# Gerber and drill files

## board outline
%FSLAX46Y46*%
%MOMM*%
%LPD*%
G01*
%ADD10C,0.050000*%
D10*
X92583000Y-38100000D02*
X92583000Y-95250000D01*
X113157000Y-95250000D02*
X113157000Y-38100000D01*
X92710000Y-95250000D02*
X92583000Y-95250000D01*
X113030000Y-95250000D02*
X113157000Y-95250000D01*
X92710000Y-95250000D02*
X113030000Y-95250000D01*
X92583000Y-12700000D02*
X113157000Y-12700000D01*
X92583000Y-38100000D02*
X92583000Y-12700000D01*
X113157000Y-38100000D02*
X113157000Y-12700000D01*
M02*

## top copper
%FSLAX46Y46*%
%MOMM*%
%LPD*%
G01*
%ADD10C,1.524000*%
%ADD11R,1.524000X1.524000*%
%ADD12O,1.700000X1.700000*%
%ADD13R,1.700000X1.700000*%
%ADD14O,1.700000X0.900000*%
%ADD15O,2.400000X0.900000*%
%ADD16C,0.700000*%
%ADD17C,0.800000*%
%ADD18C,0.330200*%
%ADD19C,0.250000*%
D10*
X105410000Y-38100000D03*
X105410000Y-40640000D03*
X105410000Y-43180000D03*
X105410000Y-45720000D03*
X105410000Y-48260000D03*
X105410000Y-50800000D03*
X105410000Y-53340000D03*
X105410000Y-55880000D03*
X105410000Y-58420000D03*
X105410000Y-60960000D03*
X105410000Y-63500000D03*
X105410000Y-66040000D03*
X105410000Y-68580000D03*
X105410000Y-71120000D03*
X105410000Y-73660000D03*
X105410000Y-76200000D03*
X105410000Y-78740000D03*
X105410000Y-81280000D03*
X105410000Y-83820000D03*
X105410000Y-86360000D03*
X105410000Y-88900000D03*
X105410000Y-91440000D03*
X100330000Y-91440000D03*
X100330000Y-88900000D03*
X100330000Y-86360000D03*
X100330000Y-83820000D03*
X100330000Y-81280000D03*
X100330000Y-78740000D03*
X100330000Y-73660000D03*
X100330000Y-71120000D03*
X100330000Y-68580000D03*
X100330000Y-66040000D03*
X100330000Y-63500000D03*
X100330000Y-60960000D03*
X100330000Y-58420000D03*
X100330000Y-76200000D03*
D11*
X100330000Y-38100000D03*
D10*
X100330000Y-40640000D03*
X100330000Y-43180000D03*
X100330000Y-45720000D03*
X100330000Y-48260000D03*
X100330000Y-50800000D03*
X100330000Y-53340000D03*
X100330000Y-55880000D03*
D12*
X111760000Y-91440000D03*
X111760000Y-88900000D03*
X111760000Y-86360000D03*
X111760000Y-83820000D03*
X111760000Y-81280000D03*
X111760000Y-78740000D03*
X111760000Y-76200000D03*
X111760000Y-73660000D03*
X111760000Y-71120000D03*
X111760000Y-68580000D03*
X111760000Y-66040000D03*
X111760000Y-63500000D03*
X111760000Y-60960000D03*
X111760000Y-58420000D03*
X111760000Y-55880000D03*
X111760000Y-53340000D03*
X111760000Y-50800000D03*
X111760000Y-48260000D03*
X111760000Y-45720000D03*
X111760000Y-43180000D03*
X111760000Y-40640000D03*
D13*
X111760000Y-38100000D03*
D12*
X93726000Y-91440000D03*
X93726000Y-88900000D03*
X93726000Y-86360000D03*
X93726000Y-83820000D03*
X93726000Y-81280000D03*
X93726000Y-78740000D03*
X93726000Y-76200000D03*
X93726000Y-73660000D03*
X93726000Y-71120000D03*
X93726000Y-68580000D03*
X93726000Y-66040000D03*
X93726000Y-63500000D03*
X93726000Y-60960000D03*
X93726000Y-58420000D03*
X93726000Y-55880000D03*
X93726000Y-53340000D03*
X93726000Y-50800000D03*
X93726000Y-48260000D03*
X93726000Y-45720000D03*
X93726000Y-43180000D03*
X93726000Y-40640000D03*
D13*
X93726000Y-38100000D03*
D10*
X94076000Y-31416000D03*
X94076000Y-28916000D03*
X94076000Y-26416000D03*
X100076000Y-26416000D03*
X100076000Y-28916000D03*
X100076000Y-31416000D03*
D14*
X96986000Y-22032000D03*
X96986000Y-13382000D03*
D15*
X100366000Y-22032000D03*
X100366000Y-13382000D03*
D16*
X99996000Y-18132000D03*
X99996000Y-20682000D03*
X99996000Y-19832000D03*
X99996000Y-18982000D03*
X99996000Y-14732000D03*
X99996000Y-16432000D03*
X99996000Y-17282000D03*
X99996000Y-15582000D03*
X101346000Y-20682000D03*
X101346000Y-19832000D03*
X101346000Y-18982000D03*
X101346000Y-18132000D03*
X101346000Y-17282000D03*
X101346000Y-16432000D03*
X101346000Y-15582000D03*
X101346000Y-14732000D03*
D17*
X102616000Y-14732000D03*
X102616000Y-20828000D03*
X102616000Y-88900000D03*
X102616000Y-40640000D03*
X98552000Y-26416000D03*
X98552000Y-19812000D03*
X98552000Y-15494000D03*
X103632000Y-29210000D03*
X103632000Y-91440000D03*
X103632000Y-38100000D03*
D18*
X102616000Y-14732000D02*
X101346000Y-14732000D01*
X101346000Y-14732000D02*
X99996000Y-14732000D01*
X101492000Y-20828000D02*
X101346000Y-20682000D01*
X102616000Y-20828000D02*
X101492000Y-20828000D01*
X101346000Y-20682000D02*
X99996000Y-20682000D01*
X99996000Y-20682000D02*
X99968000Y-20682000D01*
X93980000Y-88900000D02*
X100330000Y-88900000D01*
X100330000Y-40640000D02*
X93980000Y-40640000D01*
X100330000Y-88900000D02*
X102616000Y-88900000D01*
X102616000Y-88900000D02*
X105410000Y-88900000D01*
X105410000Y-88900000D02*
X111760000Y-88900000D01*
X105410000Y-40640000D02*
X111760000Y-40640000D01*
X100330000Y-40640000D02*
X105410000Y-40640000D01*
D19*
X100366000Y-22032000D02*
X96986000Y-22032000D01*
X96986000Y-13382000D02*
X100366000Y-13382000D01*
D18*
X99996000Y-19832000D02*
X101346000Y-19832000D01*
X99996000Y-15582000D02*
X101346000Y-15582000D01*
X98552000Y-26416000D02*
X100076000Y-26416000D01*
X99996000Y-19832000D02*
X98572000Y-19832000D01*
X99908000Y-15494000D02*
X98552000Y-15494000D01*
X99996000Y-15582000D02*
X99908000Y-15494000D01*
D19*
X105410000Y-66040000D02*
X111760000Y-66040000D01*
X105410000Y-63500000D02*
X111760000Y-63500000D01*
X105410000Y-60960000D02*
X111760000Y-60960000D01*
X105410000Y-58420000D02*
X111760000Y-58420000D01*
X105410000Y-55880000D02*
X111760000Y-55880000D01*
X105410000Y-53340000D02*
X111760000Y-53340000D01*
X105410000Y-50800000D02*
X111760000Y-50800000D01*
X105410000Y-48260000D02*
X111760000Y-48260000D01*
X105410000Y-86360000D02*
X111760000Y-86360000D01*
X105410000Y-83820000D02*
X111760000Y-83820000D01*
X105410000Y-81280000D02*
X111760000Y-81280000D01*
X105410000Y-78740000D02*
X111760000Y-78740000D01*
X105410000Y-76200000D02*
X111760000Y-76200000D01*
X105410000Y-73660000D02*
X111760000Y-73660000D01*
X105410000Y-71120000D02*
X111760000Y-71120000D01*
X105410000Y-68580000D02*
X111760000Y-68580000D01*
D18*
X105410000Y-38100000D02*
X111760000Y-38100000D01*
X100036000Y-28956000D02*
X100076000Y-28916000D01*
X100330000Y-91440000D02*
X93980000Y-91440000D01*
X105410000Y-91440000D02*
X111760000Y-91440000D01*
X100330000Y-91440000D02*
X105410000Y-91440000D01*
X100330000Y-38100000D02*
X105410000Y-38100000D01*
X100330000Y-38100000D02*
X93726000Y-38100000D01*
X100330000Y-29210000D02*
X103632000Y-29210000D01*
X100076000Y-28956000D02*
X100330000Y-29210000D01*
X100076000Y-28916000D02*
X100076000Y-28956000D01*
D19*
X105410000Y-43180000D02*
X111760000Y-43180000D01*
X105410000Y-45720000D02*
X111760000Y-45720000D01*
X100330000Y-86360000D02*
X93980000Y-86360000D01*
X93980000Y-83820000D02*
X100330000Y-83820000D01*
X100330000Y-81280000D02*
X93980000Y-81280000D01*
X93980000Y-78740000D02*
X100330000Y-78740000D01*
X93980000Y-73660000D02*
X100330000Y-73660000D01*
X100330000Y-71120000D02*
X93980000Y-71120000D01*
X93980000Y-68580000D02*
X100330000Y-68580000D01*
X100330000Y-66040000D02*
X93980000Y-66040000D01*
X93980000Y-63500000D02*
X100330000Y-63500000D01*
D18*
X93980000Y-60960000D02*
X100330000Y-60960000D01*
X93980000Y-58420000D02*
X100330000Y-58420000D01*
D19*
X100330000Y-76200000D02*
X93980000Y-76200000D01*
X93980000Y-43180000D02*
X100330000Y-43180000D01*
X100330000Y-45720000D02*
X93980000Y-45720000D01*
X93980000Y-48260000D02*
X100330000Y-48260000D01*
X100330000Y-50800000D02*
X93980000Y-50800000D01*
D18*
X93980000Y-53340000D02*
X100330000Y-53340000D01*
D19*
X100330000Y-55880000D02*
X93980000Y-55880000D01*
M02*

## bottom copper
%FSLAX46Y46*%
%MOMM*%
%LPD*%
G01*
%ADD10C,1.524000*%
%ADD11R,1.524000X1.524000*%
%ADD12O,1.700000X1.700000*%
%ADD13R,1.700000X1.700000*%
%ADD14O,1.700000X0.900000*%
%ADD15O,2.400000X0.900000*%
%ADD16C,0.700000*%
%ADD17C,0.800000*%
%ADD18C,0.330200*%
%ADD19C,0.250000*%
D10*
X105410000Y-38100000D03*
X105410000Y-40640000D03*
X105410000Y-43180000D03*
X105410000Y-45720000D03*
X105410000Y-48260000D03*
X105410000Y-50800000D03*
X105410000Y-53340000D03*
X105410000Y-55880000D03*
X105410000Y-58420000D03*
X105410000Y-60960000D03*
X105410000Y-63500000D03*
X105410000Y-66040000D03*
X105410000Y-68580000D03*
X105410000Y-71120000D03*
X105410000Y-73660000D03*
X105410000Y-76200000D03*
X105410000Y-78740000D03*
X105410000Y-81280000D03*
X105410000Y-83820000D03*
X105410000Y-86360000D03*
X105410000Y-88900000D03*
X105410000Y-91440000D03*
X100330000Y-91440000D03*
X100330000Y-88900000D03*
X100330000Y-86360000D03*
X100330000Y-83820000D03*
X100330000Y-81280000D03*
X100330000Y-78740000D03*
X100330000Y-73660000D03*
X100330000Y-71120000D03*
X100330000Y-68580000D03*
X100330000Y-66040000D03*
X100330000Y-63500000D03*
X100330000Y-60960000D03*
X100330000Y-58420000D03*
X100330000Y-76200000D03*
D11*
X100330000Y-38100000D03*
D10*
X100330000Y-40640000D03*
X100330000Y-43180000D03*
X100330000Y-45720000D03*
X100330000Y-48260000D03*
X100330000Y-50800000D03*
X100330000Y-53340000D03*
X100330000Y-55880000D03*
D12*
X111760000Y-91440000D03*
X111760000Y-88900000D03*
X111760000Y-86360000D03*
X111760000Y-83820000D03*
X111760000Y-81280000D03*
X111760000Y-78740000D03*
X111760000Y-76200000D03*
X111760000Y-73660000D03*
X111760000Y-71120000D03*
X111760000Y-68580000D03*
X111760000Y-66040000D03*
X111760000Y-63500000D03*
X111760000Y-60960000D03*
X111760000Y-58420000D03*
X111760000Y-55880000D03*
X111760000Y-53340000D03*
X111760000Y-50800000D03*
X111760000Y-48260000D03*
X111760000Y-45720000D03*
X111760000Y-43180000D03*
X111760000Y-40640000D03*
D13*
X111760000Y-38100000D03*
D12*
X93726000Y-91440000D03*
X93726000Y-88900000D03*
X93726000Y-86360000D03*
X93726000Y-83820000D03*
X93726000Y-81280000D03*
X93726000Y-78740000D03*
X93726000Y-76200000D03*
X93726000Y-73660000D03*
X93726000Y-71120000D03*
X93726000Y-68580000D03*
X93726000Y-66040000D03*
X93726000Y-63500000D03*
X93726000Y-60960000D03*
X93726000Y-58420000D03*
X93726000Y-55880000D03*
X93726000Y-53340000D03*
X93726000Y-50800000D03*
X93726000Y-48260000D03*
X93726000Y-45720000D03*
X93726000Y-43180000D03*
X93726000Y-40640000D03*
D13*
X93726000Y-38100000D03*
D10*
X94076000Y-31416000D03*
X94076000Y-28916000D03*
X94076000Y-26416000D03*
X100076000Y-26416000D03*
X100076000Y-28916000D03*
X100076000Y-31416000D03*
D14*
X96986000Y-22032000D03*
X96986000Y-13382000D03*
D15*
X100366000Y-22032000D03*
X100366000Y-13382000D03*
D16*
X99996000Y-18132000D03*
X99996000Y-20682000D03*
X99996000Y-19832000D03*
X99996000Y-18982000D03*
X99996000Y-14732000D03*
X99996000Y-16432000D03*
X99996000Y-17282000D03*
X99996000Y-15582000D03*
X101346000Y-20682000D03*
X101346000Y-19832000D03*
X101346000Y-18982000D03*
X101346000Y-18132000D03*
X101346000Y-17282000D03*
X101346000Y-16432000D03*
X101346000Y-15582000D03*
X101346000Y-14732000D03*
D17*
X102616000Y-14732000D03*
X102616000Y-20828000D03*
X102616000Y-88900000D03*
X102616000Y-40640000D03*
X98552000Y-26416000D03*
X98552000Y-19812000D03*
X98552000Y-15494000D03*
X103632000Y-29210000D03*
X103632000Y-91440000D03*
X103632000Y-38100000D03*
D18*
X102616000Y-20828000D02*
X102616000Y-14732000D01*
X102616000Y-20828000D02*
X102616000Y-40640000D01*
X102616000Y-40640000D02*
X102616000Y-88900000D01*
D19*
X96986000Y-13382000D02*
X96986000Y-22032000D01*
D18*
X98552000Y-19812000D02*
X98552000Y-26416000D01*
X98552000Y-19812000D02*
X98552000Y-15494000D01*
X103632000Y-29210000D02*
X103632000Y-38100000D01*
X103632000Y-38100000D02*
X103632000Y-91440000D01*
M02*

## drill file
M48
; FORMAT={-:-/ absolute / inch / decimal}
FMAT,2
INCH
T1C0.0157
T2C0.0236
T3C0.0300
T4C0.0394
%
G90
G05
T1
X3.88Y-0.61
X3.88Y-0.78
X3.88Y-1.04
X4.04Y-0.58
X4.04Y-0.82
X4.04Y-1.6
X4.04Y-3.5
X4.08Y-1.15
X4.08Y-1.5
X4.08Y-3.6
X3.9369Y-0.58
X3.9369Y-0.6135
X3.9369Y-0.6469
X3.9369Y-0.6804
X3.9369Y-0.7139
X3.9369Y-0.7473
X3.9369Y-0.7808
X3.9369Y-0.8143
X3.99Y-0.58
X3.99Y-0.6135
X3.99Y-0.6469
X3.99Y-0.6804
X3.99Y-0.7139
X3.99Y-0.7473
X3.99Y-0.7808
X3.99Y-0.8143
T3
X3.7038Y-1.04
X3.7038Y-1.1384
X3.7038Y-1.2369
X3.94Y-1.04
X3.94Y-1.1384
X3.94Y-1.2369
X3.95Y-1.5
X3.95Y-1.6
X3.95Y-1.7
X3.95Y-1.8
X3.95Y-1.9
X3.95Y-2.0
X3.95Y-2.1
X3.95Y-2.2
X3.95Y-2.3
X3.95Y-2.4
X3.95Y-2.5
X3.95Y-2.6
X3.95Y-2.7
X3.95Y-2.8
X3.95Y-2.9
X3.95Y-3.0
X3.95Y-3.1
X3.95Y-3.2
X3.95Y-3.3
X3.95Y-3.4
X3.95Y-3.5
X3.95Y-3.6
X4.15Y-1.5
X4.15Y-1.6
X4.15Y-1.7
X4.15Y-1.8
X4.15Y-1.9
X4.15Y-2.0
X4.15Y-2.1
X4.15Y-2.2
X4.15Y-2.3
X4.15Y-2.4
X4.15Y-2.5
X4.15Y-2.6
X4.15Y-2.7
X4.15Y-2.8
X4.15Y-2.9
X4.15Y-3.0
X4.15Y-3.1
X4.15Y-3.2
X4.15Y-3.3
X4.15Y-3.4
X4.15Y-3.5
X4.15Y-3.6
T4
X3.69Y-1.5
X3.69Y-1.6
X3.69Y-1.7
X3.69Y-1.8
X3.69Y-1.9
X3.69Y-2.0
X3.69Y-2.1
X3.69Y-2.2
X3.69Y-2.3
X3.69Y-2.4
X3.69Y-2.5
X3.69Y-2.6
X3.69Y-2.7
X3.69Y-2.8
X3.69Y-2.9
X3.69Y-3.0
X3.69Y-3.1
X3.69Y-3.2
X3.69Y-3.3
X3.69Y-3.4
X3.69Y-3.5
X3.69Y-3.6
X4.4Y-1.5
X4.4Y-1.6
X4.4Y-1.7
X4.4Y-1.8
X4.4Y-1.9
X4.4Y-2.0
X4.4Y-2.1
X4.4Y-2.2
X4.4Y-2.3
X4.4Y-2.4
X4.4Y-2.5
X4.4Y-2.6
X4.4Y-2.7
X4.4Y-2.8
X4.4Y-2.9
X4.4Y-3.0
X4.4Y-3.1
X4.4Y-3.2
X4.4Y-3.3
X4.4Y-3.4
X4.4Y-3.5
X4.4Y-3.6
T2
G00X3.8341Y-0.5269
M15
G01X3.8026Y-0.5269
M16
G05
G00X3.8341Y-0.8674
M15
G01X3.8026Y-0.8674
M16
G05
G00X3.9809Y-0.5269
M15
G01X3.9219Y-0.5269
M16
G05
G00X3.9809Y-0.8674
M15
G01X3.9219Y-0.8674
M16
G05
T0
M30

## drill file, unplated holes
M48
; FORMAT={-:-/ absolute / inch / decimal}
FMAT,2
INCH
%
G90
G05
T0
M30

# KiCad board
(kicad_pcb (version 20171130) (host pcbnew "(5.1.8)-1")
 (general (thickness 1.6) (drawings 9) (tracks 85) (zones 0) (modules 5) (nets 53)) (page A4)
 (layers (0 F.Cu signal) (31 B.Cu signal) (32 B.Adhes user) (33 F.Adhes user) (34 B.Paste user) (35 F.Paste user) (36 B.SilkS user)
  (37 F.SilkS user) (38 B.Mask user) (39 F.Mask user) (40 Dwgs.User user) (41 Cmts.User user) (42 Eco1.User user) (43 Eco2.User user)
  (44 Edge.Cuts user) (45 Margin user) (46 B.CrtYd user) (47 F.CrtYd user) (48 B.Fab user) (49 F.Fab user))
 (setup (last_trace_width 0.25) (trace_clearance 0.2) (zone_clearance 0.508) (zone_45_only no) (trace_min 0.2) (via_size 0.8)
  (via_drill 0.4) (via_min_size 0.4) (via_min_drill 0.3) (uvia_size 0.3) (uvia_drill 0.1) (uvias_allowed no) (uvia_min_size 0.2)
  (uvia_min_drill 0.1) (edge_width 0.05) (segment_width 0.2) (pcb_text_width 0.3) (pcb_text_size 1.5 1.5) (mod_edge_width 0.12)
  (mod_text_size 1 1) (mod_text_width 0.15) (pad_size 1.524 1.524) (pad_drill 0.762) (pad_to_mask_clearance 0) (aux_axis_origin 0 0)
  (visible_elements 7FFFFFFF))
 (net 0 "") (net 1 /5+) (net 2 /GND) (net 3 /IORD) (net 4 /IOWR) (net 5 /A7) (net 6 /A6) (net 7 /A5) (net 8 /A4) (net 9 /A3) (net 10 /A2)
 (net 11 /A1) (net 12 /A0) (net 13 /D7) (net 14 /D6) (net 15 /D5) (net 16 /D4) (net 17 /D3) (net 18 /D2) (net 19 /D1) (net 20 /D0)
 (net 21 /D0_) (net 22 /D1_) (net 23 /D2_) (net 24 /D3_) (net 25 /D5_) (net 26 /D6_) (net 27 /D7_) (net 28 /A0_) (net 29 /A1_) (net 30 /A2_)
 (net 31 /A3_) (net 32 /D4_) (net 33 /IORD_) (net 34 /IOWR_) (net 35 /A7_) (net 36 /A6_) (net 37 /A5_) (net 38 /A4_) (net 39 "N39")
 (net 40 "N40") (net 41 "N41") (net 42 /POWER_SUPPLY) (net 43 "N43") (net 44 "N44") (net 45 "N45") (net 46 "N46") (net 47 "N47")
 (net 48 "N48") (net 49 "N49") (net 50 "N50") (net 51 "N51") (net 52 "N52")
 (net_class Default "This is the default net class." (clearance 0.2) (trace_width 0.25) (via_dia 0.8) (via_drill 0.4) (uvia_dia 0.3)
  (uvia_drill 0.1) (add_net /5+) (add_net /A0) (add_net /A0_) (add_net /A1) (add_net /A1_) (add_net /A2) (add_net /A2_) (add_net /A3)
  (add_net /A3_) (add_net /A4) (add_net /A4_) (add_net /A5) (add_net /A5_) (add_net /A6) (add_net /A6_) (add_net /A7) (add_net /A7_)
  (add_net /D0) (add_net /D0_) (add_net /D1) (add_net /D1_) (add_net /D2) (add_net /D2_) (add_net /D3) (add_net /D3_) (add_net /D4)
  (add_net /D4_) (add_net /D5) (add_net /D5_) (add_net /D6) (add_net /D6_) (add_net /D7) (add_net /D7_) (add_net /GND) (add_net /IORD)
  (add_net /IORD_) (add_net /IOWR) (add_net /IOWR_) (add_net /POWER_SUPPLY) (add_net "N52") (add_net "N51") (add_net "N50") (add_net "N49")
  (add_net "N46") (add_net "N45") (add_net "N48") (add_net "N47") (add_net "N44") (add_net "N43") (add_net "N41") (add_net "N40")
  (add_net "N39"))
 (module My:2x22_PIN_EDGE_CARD (layer F.Cu) (at 100.33 38.1)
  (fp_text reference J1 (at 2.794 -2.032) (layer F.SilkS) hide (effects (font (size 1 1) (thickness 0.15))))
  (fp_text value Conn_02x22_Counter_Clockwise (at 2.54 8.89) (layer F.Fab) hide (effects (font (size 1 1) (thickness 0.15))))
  (pad 44 thru_hole circle (at 5.08 0) (size 1.524 1.524) (drill 0.762) (layers *.Cu *.Mask) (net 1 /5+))
  (pad 43 thru_hole circle (at 5.08 2.54) (size 1.524 1.524) (drill 0.762) (layers *.Cu *.Mask) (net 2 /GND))
  (pad 42 thru_hole circle (at 5.08 5.08) (size 1.524 1.524) (drill 0.762) (layers *.Cu *.Mask) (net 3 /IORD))
  (pad 41 thru_hole circle (at 5.08 7.62) (size 1.524 1.524) (drill 0.762) (layers *.Cu *.Mask) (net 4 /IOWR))
  (pad 40 thru_hole circle (at 5.08 10.16) (size 1.524 1.524) (drill 0.762) (layers *.Cu *.Mask) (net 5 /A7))
  (pad 39 thru_hole circle (at 5.08 12.7) (size 1.524 1.524) (drill 0.762) (layers *.Cu *.Mask) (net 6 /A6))
  (pad 38 thru_hole circle (at 5.08 15.24) (size 1.524 1.524) (drill 0.762) (layers *.Cu *.Mask) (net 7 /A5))
  (pad 37 thru_hole circle (at 5.08 17.78) (size 1.524 1.524) (drill 0.762) (layers *.Cu *.Mask) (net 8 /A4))
  (pad 36 thru_hole circle (at 5.08 20.32) (size 1.524 1.524) (drill 0.762) (layers *.Cu *.Mask) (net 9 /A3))
  (pad 35 thru_hole circle (at 5.08 22.86) (size 1.524 1.524) (drill 0.762) (layers *.Cu *.Mask) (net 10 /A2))
  (pad 34 thru_hole circle (at 5.08 25.4) (size 1.524 1.524) (drill 0.762) (layers *.Cu *.Mask) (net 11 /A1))
  (pad 33 thru_hole circle (at 5.08 27.94) (size 1.524 1.524) (drill 0.762) (layers *.Cu *.Mask) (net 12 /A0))
  (pad 32 thru_hole circle (at 5.08 30.48) (size 1.524 1.524) (drill 0.762) (layers *.Cu *.Mask) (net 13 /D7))
  (pad 31 thru_hole circle (at 5.08 33.02) (size 1.524 1.524) (drill 0.762) (layers *.Cu *.Mask) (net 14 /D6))
  (pad 30 thru_hole circle (at 5.08 35.56) (size 1.524 1.524) (drill 0.762) (layers *.Cu *.Mask) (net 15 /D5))
  (pad 29 thru_hole circle (at 5.08 38.1) (size 1.524 1.524) (drill 0.762) (layers *.Cu *.Mask) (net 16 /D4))
  (pad 28 thru_hole circle (at 5.08 40.64) (size 1.524 1.524) (drill 0.762) (layers *.Cu *.Mask) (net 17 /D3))
  (pad 27 thru_hole circle (at 5.08 43.18) (size 1.524 1.524) (drill 0.762) (layers *.Cu *.Mask) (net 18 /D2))
  (pad 26 thru_hole circle (at 5.08 45.72) (size 1.524 1.524) (drill 0.762) (layers *.Cu *.Mask) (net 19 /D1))
  (pad 25 thru_hole circle (at 5.08 48.26) (size 1.524 1.524) (drill 0.762) (layers *.Cu *.Mask) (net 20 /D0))
  (pad 24 thru_hole circle (at 5.08 50.8) (size 1.524 1.524) (drill 0.762) (layers *.Cu *.Mask) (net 2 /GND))
  (pad 23 thru_hole circle (at 5.08 53.34) (size 1.524 1.524) (drill 0.762) (layers *.Cu *.Mask) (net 1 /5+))
  (pad 22 thru_hole circle (at 0 53.34) (size 1.524 1.524) (drill 0.762) (layers *.Cu *.Mask) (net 1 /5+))
  (pad 21 thru_hole circle (at 0 50.8) (size 1.524 1.524) (drill 0.762) (layers *.Cu *.Mask) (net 2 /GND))
  (pad 20 thru_hole circle (at 0 48.26) (size 1.524 1.524) (drill 0.762) (layers *.Cu *.Mask) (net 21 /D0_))
  (pad 19 thru_hole circle (at 0 45.72) (size 1.524 1.524) (drill 0.762) (layers *.Cu *.Mask) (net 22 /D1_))
  (pad 18 thru_hole circle (at 0 43.18) (size 1.524 1.524) (drill 0.762) (layers *.Cu *.Mask) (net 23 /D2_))
  (pad 17 thru_hole circle (at 0 40.64) (size 1.524 1.524) (drill 0.762) (layers *.Cu *.Mask) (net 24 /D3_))
  (pad 15 thru_hole circle (at 0 35.56) (size 1.524 1.524) (drill 0.762) (layers *.Cu *.Mask) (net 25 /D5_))
  (pad 14 thru_hole circle (at 0 33.02) (size 1.524 1.524) (drill 0.762) (layers *.Cu *.Mask) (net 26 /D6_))
  (pad 13 thru_hole circle (at 0 30.48) (size 1.524 1.524) (drill 0.762) (layers *.Cu *.Mask) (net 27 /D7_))
  (pad 12 thru_hole circle (at 0 27.94) (size 1.524 1.524) (drill 0.762) (layers *.Cu *.Mask) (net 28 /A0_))
  (pad 11 thru_hole circle (at 0 25.4) (size 1.524 1.524) (drill 0.762) (layers *.Cu *.Mask) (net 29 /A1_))
  (pad 10 thru_hole circle (at 0 22.86) (size 1.524 1.524) (drill 0.762) (layers *.Cu *.Mask) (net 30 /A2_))
  (pad 9 thru_hole circle (at 0 20.32) (size 1.524 1.524) (drill 0.762) (layers *.Cu *.Mask) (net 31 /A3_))
  (pad 16 thru_hole circle (at 0 38.1 180) (size 1.524 1.524) (drill 0.762) (layers *.Cu *.Mask) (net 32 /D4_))
  (pad 1 thru_hole rect (at 0 0) (size 1.524 1.524) (drill 0.762) (layers *.Cu *.Mask) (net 1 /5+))
  (pad 2 thru_hole circle (at 0 2.54) (size 1.524 1.524) (drill 0.762) (layers *.Cu *.Mask) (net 2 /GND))
  (pad 3 thru_hole circle (at 0 5.08) (size 1.524 1.524) (drill 0.762) (layers *.Cu *.Mask) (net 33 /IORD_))
  (pad 4 thru_hole circle (at 0 7.62) (size 1.524 1.524) (drill 0.762) (layers *.Cu *.Mask) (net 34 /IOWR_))
  (pad 5 thru_hole circle (at 0 10.16) (size 1.524 1.524) (drill 0.762) (layers *.Cu *.Mask) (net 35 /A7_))
  (pad 6 thru_hole circle (at 0 12.7) (size 1.524 1.524) (drill 0.762) (layers *.Cu *.Mask) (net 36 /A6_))
  (pad 7 thru_hole circle (at 0 15.24) (size 1.524 1.524) (drill 0.762) (layers *.Cu *.Mask) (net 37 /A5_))
  (pad 8 thru_hole circle (at 0 17.78 180) (size 1.524 1.524) (drill 0.762) (layers *.Cu *.Mask) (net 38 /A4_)))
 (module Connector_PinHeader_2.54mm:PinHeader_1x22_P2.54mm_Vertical (layer F.Cu) (at 111.76 38.1)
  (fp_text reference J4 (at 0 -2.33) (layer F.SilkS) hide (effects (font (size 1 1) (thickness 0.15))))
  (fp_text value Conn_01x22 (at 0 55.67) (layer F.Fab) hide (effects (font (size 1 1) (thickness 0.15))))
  (pad 22 thru_hole oval (at 0 53.34) (size 1.7 1.7) (drill 1) (layers *.Cu *.Mask) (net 1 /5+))
  (pad 21 thru_hole oval (at 0 50.8) (size 1.7 1.7) (drill 1) (layers *.Cu *.Mask) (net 2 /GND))
  (pad 20 thru_hole oval (at 0 48.26) (size 1.7 1.7) (drill 1) (layers *.Cu *.Mask) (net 20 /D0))
  (pad 19 thru_hole oval (at 0 45.72) (size 1.7 1.7) (drill 1) (layers *.Cu *.Mask) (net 19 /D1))
  (pad 18 thru_hole oval (at 0 43.18) (size 1.7 1.7) (drill 1) (layers *.Cu *.Mask) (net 18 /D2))
  (pad 17 thru_hole oval (at 0 40.64) (size 1.7 1.7) (drill 1) (layers *.Cu *.Mask) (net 17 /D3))
  (pad 16 thru_hole oval (at 0 38.1) (size 1.7 1.7) (drill 1) (layers *.Cu *.Mask) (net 16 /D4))
  (pad 15 thru_hole oval (at 0 35.56) (size 1.7 1.7) (drill 1) (layers *.Cu *.Mask) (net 15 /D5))
  (pad 14 thru_hole oval (at 0 33.02) (size 1.7 1.7) (drill 1) (layers *.Cu *.Mask) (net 14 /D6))
  (pad 13 thru_hole oval (at 0 30.48) (size 1.7 1.7) (drill 1) (layers *.Cu *.Mask) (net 13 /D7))
  (pad 12 thru_hole oval (at 0 27.94) (size 1.7 1.7) (drill 1) (layers *.Cu *.Mask) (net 12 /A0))
  (pad 11 thru_hole oval (at 0 25.4) (size 1.7 1.7) (drill 1) (layers *.Cu *.Mask) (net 11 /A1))
  (pad 10 thru_hole oval (at 0 22.86) (size 1.7 1.7) (drill 1) (layers *.Cu *.Mask) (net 10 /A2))
  (pad 9 thru_hole oval (at 0 20.32) (size 1.7 1.7) (drill 1) (layers *.Cu *.Mask) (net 9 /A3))
  (pad 8 thru_hole oval (at 0 17.78) (size 1.7 1.7) (drill 1) (layers *.Cu *.Mask) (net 8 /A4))
  (pad 7 thru_hole oval (at 0 15.24) (size 1.7 1.7) (drill 1) (layers *.Cu *.Mask) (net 7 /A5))
  (pad 6 thru_hole oval (at 0 12.7) (size 1.7 1.7) (drill 1) (layers *.Cu *.Mask) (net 6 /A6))
  (pad 5 thru_hole oval (at 0 10.16) (size 1.7 1.7) (drill 1) (layers *.Cu *.Mask) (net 5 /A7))
  (pad 4 thru_hole oval (at 0 7.62) (size 1.7 1.7) (drill 1) (layers *.Cu *.Mask) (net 4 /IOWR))
  (pad 3 thru_hole oval (at 0 5.08) (size 1.7 1.7) (drill 1) (layers *.Cu *.Mask) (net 3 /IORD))
  (pad 2 thru_hole oval (at 0 2.54) (size 1.7 1.7) (drill 1) (layers *.Cu *.Mask) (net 2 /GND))
  (pad 1 thru_hole rect (at 0 0) (size 1.7 1.7) (drill 1) (layers *.Cu *.Mask) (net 1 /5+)))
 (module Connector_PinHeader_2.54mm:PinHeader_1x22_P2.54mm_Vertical (layer F.Cu) (at 93.726 38.1)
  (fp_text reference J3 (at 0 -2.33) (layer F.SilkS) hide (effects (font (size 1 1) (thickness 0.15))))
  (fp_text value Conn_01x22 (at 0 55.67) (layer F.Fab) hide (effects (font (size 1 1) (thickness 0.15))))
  (pad 22 thru_hole oval (at 0 53.34) (size 1.7 1.7) (drill 1) (layers *.Cu *.Mask) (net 1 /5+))
  (pad 21 thru_hole oval (at 0 50.8) (size 1.7 1.7) (drill 1) (layers *.Cu *.Mask) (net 2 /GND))
  (pad 20 thru_hole oval (at 0 48.26) (size 1.7 1.7) (drill 1) (layers *.Cu *.Mask) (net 21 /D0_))
  (pad 19 thru_hole oval (at 0 45.72) (size 1.7 1.7) (drill 1) (layers *.Cu *.Mask) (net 22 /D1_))
  (pad 18 thru_hole oval (at 0 43.18) (size 1.7 1.7) (drill 1) (layers *.Cu *.Mask) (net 23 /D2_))
  (pad 17 thru_hole oval (at 0 40.64) (size 1.7 1.7) (drill 1) (layers *.Cu *.Mask) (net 24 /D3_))
  (pad 16 thru_hole oval (at 0 38.1) (size 1.7 1.7) (drill 1) (layers *.Cu *.Mask) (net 32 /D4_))
  (pad 15 thru_hole oval (at 0 35.56) (size 1.7 1.7) (drill 1) (layers *.Cu *.Mask) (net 25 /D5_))
  (pad 14 thru_hole oval (at 0 33.02) (size 1.7 1.7) (drill 1) (layers *.Cu *.Mask) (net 26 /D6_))
  (pad 13 thru_hole oval (at 0 30.48) (size 1.7 1.7) (drill 1) (layers *.Cu *.Mask) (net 27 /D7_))
  (pad 12 thru_hole oval (at 0 27.94) (size 1.7 1.7) (drill 1) (layers *.Cu *.Mask) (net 28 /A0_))
  (pad 11 thru_hole oval (at 0 25.4) (size 1.7 1.7) (drill 1) (layers *.Cu *.Mask) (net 29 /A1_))
  (pad 10 thru_hole oval (at 0 22.86) (size 1.7 1.7) (drill 1) (layers *.Cu *.Mask) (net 30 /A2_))
  (pad 9 thru_hole oval (at 0 20.32) (size 1.7 1.7) (drill 1) (layers *.Cu *.Mask) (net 31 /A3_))
  (pad 8 thru_hole oval (at 0 17.78) (size 1.7 1.7) (drill 1) (layers *.Cu *.Mask) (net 38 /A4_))
  (pad 7 thru_hole oval (at 0 15.24) (size 1.7 1.7) (drill 1) (layers *.Cu *.Mask) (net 37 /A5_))
  (pad 6 thru_hole oval (at 0 12.7) (size 1.7 1.7) (drill 1) (layers *.Cu *.Mask) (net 36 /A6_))
  (pad 5 thru_hole oval (at 0 10.16) (size 1.7 1.7) (drill 1) (layers *.Cu *.Mask) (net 35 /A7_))
  (pad 4 thru_hole oval (at 0 7.62) (size 1.7 1.7) (drill 1) (layers *.Cu *.Mask) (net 34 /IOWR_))
  (pad 3 thru_hole oval (at 0 5.08) (size 1.7 1.7) (drill 1) (layers *.Cu *.Mask) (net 33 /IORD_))
  (pad 2 thru_hole oval (at 0 2.54) (size 1.7 1.7) (drill 1) (layers *.Cu *.Mask) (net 2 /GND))
  (pad 1 thru_hole rect (at 0 0) (size 1.7 1.7) (drill 1) (layers *.Cu *.Mask) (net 1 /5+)))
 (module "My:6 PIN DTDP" (layer F.Cu) (at 100.076 31.416 180)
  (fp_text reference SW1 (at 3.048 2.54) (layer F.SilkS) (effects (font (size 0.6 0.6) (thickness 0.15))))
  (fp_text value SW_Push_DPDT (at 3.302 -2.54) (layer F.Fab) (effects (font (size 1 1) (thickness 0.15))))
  (pad 6 thru_hole circle (at 6 0 180) (size 1.524 1.524) (drill 0.762) (layers *.Cu *.Mask) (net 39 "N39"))
  (pad 5 thru_hole circle (at 6 2.5 180) (size 1.524 1.524) (drill 0.762) (layers *.Cu *.Mask) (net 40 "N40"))
  (pad 4 thru_hole circle (at 6 5 180) (size 1.524 1.524) (drill 0.762) (layers *.Cu *.Mask) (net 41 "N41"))
  (pad 3 thru_hole circle (at 0 5 180) (size 1.524 1.524) (drill 0.762) (layers *.Cu *.Mask) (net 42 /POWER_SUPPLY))
  (pad 2 thru_hole circle (at 0 2.5 180) (size 1.524 1.524) (drill 0.762) (layers *.Cu *.Mask) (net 1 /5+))
  (pad 1 thru_hole circle (at 0 0 180) (size 1.524 1.524) (drill 0.762) (layers *.Cu *.Mask) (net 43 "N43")))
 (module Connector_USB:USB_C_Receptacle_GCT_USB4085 (layer F.Cu) (at 101.346 14.732 270)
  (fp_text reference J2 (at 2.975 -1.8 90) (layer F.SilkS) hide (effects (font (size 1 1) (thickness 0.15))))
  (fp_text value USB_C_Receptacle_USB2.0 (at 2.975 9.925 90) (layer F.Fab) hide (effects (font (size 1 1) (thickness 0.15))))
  (pad S1 thru_hole oval (at 7.3 4.36 270) (size 0.9 1.7) (drill oval 0.6 1.4) (layers *.Cu *.Mask) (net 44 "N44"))
  (pad S1 thru_hole oval (at -1.35 4.36 270) (size 0.9 1.7) (drill oval 0.6 1.4) (layers *.Cu *.Mask) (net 44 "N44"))
  (pad S1 thru_hole oval (at 7.3 0.98 270) (size 0.9 2.4) (drill oval 0.6 2.1) (layers *.Cu *.Mask) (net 44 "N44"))
  (pad S1 thru_hole oval (at -1.35 0.98 270) (size 0.9 2.4) (drill oval 0.6 2.1) (layers *.Cu *.Mask) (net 44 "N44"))
  (pad B6 thru_hole circle (at 3.4 1.35 270) (size 0.7 0.7) (drill 0.4) (layers *.Cu *.Mask) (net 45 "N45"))
  (pad B1 thru_hole circle (at 5.95 1.35 270) (size 0.7 0.7) (drill 0.4) (layers *.Cu *.Mask) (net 2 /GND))
  (pad B4 thru_hole circle (at 5.1 1.35 270) (size 0.7 0.7) (drill 0.4) (layers *.Cu *.Mask) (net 42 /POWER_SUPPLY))
  (pad B5 thru_hole circle (at 4.25 1.35 270) (size 0.7 0.7) (drill 0.4) (layers *.Cu *.Mask) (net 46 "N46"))
  (pad B12 thru_hole circle (at 0 1.35 270) (size 0.7 0.7) (drill 0.4) (layers *.Cu *.Mask) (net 2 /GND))
  (pad B8 thru_hole circle (at 1.7 1.35 270) (size 0.7 0.7) (drill 0.4) (layers *.Cu *.Mask) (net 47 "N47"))
  (pad B7 thru_hole circle (at 2.55 1.35 270) (size 0.7 0.7) (drill 0.4) (layers *.Cu *.Mask) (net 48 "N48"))
  (pad B9 thru_hole circle (at 0.85 1.35 270) (size 0.7 0.7) (drill 0.4) (layers *.Cu *.Mask) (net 42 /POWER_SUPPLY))
  (pad A12 thru_hole circle (at 5.95 0 270) (size 0.7 0.7) (drill 0.4) (layers *.Cu *.Mask) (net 2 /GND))
  (pad A9 thru_hole circle (at 5.1 0 270) (size 0.7 0.7) (drill 0.4) (layers *.Cu *.Mask) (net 42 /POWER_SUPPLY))
  (pad A8 thru_hole circle (at 4.25 0 270) (size 0.7 0.7) (drill 0.4) (layers *.Cu *.Mask) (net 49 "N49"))
  (pad A7 thru_hole circle (at 3.4 0 270) (size 0.7 0.7) (drill 0.4) (layers *.Cu *.Mask) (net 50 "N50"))
  (pad A6 thru_hole circle (at 2.55 0 270) (size 0.7 0.7) (drill 0.4) (layers *.Cu *.Mask) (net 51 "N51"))
  (pad A5 thru_hole circle (at 1.7 0 270) (size 0.7 0.7) (drill 0.4) (layers *.Cu *.Mask) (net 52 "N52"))
  (pad A4 thru_hole circle (at 0.85 0 270) (size 0.7 0.7) (drill 0.4) (layers *.Cu *.Mask) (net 42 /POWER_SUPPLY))
  (pad A1 thru_hole circle (at 0 0 270) (size 0.7 0.7) (drill 0.4) (layers *.Cu *.Mask) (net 2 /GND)))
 (gr_line (start 92.583 38.1) (end 92.583 95.25) (layer Edge.Cuts) (width 0.05))
 (gr_line (start 113.157 95.25) (end 113.157 38.1) (layer Edge.Cuts) (width 0.05))
 (gr_line (start 92.71 95.25) (end 92.583 95.25) (layer Edge.Cuts) (width 0.05))
 (gr_line (start 113.03 95.25) (end 113.157 95.25) (layer Edge.Cuts) (width 0.05))
 (gr_line (start 92.71 95.25) (end 113.03 95.25) (layer Edge.Cuts) (width 0.05))
 (gr_line (start 92.583 12.7) (end 113.157 12.7) (layer Edge.Cuts) (width 0.05))
 (gr_line (start 92.583 38.1) (end 92.583 12.7) (layer Edge.Cuts) (width 0.05))
 (gr_line (start 113.157 38.1) (end 113.157 12.7) (layer Edge.Cuts) (width 0.05))
 (via (at 102.616 14.732) (size 0.8) (drill 0.4) (layers F.Cu B.Cu) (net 2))
 (segment (start 102.616 14.732) (end 101.346 14.732) (width 0.3302) (layer F.Cu) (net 2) (status 20))
 (segment (start 101.346 14.732) (end 99.996 14.732) (width 0.3302) (layer F.Cu) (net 2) (status 30))
 (segment (start 102.616 20.828) (end 102.616 14.732) (width 0.3302) (layer B.Cu) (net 2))
 (via (at 102.616 20.828) (size 0.8) (drill 0.4) (layers F.Cu B.Cu) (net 2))
 (segment (start 101.492 20.828) (end 101.346 20.682) (width 0.3302) (layer F.Cu) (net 2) (status 30))
 (segment (start 102.616 20.828) (end 101.492 20.828) (width 0.3302) (layer F.Cu) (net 2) (status 20))
 (segment (start 101.346 20.682) (end 99.996 20.682) (width 0.3302) (layer F.Cu) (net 2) (status 30))
 (segment (start 99.996 20.682) (end 99.968 20.682) (width 0.3302) (layer F.Cu) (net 2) (status 30))
 (segment (start 100.366 22.032) (end 96.986 22.032) (width 0.25) (layer F.Cu) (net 44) (status 30))
 (segment (start 96.986 13.382) (end 100.366 13.382) (width 0.25) (layer F.Cu) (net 44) (status 30))
 (segment (start 96.986 13.382) (end 96.986 22.032) (width 0.25) (layer B.Cu) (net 44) (status 30))
 (segment (start 99.996 19.832) (end 101.346 19.832) (width 0.3302) (layer F.Cu) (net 42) (status 30))
 (segment (start 99.996 15.582) (end 101.346 15.582) (width 0.3302) (layer F.Cu) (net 42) (status 30))
 (via (at 98.552 26.416) (size 0.8) (drill 0.4) (layers F.Cu B.Cu) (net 42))
 (segment (start 98.552 26.416) (end 100.076 26.416) (width 0.3302) (layer F.Cu) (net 42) (status 20))
 (segment (start 99.996 19.832) (end 98.572 19.832) (width 0.3302) (layer F.Cu) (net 42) (status 10))
 (segment (start 98.552 19.812) (end 98.552 26.416) (width 0.3302) (layer B.Cu) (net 42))
 (via (at 98.552 19.812) (size 0.8) (drill 0.4) (layers F.Cu B.Cu) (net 42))
 (segment (start 98.552 19.812) (end 98.552 15.494) (width 0.3302) (layer B.Cu) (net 42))
 (via (at 98.552 15.494) (size 0.8) (drill 0.4) (layers F.Cu B.Cu) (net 42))
 (segment (start 99.908 15.494) (end 98.552 15.494) (width 0.3302) (layer F.Cu) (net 42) (status 10))
 (segment (start 99.996 15.582) (end 99.908 15.494) (width 0.3302) (layer F.Cu) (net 42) (status 30))
 (segment (start 105.41 38.1) (end 111.76 38.1) (width 0.3302) (layer F.Cu) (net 1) (status 30))
 (segment (start 100.036 28.956) (end 100.076 28.916) (width 0.3302) (layer F.Cu) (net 1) (status 30))
 (segment (start 100.33 91.44) (end 93.98 91.44) (width 0.3302) (layer F.Cu) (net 1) (status 30))
 (segment (start 93.98 88.9) (end 100.33 88.9) (width 0.3302) (layer F.Cu) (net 2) (status 30))
 (segment (start 100.33 86.36) (end 93.98 86.36) (width 0.25) (layer F.Cu) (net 21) (status 30))
 (segment (start 93.98 83.82) (end 100.33 83.82) (width 0.25) (layer F.Cu) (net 22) (status 30))
 (segment (start 100.33 81.28) (end 93.98 81.28) (width 0.25) (layer F.Cu) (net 23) (status 30))
 (segment (start 93.98 78.74) (end 100.33 78.74) (width 0.25) (layer F.Cu) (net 24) (status 30))
 (segment (start 100.33 76.2) (end 93.98 76.2) (width 0.25) (layer F.Cu) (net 32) (status 30))
 (segment (start 93.98 73.66) (end 100.33 73.66) (width 0.25) (layer F.Cu) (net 25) (status 30))
 (segment (start 100.33 71.12) (end 93.98 71.12) (width 0.25) (layer F.Cu) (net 26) (status 30))
 (segment (start 93.98 68.58) (end 100.33 68.58) (width 0.25) (layer F.Cu) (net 27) (status 30))
 (segment (start 100.33 66.04) (end 93.98 66.04) (width 0.25) (layer F.Cu) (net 28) (status 30))
 (segment (start 93.98 63.5) (end 100.33 63.5) (width 0.25) (layer F.Cu) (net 29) (status 30))
 (segment (start 93.98 58.42) (end 100.33 58.42) (width 0.3302) (layer F.Cu) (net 31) (status 30))
 (segment (start 100.33 55.88) (end 93.98 55.88) (width 0.25) (layer F.Cu) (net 38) (status 30))
 (segment (start 93.98 53.34) (end 100.33 53.34) (width 0.3302) (layer F.Cu) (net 37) (status 30))
 (segment (start 100.33 50.8) (end 93.98 50.8) (width 0.25) (layer F.Cu) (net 36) (status 30))
 (segment (start 93.98 48.26) (end 100.33 48.26) (width 0.25) (layer F.Cu) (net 35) (status 30))
 (segment (start 100.33 45.72) (end 93.98 45.72) (width 0.25) (layer F.Cu) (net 34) (status 30))
 (segment (start 100.33 40.64) (end 93.98 40.64) (width 0.3302) (layer F.Cu) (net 2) (status 30))
 (segment (start 102.616 20.828) (end 102.616 40.64) (width 0.3302) (layer B.Cu) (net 2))
 (via (at 102.616 88.9) (size 0.8) (drill 0.4) (layers F.Cu B.Cu) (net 2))
 (segment (start 100.33 88.9) (end 102.616 88.9) (width 0.3302) (layer F.Cu) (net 2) (status 10))
 (segment (start 102.616 88.9) (end 105.41 88.9) (width 0.3302) (layer F.Cu) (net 2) (status 20))
 (segment (start 105.41 88.9) (end 111.76 88.9) (width 0.3302) (layer F.Cu) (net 2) (status 30))
 (segment (start 105.41 86.36) (end 111.76 86.36) (width 0.25) (layer F.Cu) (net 20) (status 30))
 (segment (start 105.41 78.74) (end 111.76 78.74) (width 0.25) (layer F.Cu) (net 17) (status 30))
 (segment (start 105.41 83.82) (end 111.76 83.82) (width 0.25) (layer F.Cu) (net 19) (status 30))
 (segment (start 105.41 76.2) (end 111.76 76.2) (width 0.25) (layer F.Cu) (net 16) (status 30))
 (segment (start 105.41 81.28) (end 111.76 81.28) (width 0.25) (layer F.Cu) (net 18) (status 30))
 (segment (start 105.41 71.12) (end 111.76 71.12) (width 0.25) (layer F.Cu) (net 14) (status 30))
 (segment (start 105.41 68.58) (end 111.76 68.58) (width 0.25) (layer F.Cu) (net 13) (status 30))
 (segment (start 105.41 73.66) (end 111.76 73.66) (width 0.25) (layer F.Cu) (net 15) (status 30))
 (segment (start 105.41 66.04) (end 111.76 66.04) (width 0.25) (layer F.Cu) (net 12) (status 30))
 (segment (start 105.41 58.42) (end 111.76 58.42) (width 0.25) (layer F.Cu) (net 9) (status 30))
 (segment (start 105.41 63.5) (end 111.76 63.5) (width 0.25) (layer F.Cu) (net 11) (status 30))
 (segment (start 105.41 55.88) (end 111.76 55.88) (width 0.25) (layer F.Cu) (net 8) (status 30))
 (segment (start 105.41 60.96) (end 111.76 60.96) (width 0.25) (layer F.Cu) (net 10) (status 30))
 (segment (start 105.41 48.26) (end 111.76 48.26) (width 0.25) (layer F.Cu) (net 5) (status 30))
 (segment (start 105.41 53.34) (end 111.76 53.34) (width 0.25) (layer F.Cu) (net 7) (status 30))
 (segment (start 105.41 45.72) (end 111.76 45.72) (width 0.25) (layer F.Cu) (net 4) (status 30))
 (segment (start 105.41 50.8) (end 111.76 50.8) (width 0.25) (layer F.Cu) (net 6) (status 30))
 (segment (start 105.41 40.64) (end 111.76 40.64) (width 0.3302) (layer F.Cu) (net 2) (status 30))
 (segment (start 100.33 40.64) (end 105.41 40.64) (width 0.3302) (layer F.Cu) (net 2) (status 30))
 (segment (start 102.616 40.64) (end 102.616 88.9) (width 0.3302) (layer B.Cu) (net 2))
 (via (at 102.616 40.64) (size 0.8) (drill 0.4) (layers F.Cu B.Cu) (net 2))
 (segment (start 105.41 43.18) (end 111.76 43.18) (width 0.25) (layer F.Cu) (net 3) (status 30))
 (segment (start 105.41 91.44) (end 111.76 91.44) (width 0.3302) (layer F.Cu) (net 1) (status 30))
 (segment (start 100.33 91.44) (end 105.41 91.44) (width 0.3302) (layer F.Cu) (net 1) (status 30))
 (segment (start 93.98 43.18) (end 100.33 43.18) (width 0.25) (layer F.Cu) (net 33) (status 30))
 (segment (start 100.33 38.1) (end 105.41 38.1) (width 0.3302) (layer F.Cu) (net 1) (status 30))
 (segment (start 100.33 38.1) (end 93.726 38.1) (width 0.3302) (layer F.Cu) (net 1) (status 30))
 (segment (start 100.33 29.21) (end 103.632 29.21) (width 0.3302) (layer F.Cu) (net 1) (status 10))
 (segment (start 100.076 28.956) (end 100.33 29.21) (width 0.3302) (layer F.Cu) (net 1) (status 30))
 (segment (start 100.076 28.916) (end 100.076 28.956) (width 0.3302) (layer F.Cu) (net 1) (status 30))
 (via (at 103.632 29.21) (size 0.8) (drill 0.4) (layers F.Cu B.Cu) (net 1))
 (segment (start 103.632 29.21) (end 103.632 38.1) (width 0.3302) (layer B.Cu) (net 1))
 (segment (start 103.632 38.1) (end 103.632 91.44) (width 0.3302) (layer B.Cu) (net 1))
 (via (at 103.632 91.44) (size 0.8) (drill 0.4) (layers F.Cu B.Cu) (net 1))
 (via (at 103.632 38.1) (size 0.8) (drill 0.4) (layers F.Cu B.Cu) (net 1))
 (segment (start 93.98 60.96) (end 100.33 60.96) (width 0.3302) (layer F.Cu) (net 30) (status 30)))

